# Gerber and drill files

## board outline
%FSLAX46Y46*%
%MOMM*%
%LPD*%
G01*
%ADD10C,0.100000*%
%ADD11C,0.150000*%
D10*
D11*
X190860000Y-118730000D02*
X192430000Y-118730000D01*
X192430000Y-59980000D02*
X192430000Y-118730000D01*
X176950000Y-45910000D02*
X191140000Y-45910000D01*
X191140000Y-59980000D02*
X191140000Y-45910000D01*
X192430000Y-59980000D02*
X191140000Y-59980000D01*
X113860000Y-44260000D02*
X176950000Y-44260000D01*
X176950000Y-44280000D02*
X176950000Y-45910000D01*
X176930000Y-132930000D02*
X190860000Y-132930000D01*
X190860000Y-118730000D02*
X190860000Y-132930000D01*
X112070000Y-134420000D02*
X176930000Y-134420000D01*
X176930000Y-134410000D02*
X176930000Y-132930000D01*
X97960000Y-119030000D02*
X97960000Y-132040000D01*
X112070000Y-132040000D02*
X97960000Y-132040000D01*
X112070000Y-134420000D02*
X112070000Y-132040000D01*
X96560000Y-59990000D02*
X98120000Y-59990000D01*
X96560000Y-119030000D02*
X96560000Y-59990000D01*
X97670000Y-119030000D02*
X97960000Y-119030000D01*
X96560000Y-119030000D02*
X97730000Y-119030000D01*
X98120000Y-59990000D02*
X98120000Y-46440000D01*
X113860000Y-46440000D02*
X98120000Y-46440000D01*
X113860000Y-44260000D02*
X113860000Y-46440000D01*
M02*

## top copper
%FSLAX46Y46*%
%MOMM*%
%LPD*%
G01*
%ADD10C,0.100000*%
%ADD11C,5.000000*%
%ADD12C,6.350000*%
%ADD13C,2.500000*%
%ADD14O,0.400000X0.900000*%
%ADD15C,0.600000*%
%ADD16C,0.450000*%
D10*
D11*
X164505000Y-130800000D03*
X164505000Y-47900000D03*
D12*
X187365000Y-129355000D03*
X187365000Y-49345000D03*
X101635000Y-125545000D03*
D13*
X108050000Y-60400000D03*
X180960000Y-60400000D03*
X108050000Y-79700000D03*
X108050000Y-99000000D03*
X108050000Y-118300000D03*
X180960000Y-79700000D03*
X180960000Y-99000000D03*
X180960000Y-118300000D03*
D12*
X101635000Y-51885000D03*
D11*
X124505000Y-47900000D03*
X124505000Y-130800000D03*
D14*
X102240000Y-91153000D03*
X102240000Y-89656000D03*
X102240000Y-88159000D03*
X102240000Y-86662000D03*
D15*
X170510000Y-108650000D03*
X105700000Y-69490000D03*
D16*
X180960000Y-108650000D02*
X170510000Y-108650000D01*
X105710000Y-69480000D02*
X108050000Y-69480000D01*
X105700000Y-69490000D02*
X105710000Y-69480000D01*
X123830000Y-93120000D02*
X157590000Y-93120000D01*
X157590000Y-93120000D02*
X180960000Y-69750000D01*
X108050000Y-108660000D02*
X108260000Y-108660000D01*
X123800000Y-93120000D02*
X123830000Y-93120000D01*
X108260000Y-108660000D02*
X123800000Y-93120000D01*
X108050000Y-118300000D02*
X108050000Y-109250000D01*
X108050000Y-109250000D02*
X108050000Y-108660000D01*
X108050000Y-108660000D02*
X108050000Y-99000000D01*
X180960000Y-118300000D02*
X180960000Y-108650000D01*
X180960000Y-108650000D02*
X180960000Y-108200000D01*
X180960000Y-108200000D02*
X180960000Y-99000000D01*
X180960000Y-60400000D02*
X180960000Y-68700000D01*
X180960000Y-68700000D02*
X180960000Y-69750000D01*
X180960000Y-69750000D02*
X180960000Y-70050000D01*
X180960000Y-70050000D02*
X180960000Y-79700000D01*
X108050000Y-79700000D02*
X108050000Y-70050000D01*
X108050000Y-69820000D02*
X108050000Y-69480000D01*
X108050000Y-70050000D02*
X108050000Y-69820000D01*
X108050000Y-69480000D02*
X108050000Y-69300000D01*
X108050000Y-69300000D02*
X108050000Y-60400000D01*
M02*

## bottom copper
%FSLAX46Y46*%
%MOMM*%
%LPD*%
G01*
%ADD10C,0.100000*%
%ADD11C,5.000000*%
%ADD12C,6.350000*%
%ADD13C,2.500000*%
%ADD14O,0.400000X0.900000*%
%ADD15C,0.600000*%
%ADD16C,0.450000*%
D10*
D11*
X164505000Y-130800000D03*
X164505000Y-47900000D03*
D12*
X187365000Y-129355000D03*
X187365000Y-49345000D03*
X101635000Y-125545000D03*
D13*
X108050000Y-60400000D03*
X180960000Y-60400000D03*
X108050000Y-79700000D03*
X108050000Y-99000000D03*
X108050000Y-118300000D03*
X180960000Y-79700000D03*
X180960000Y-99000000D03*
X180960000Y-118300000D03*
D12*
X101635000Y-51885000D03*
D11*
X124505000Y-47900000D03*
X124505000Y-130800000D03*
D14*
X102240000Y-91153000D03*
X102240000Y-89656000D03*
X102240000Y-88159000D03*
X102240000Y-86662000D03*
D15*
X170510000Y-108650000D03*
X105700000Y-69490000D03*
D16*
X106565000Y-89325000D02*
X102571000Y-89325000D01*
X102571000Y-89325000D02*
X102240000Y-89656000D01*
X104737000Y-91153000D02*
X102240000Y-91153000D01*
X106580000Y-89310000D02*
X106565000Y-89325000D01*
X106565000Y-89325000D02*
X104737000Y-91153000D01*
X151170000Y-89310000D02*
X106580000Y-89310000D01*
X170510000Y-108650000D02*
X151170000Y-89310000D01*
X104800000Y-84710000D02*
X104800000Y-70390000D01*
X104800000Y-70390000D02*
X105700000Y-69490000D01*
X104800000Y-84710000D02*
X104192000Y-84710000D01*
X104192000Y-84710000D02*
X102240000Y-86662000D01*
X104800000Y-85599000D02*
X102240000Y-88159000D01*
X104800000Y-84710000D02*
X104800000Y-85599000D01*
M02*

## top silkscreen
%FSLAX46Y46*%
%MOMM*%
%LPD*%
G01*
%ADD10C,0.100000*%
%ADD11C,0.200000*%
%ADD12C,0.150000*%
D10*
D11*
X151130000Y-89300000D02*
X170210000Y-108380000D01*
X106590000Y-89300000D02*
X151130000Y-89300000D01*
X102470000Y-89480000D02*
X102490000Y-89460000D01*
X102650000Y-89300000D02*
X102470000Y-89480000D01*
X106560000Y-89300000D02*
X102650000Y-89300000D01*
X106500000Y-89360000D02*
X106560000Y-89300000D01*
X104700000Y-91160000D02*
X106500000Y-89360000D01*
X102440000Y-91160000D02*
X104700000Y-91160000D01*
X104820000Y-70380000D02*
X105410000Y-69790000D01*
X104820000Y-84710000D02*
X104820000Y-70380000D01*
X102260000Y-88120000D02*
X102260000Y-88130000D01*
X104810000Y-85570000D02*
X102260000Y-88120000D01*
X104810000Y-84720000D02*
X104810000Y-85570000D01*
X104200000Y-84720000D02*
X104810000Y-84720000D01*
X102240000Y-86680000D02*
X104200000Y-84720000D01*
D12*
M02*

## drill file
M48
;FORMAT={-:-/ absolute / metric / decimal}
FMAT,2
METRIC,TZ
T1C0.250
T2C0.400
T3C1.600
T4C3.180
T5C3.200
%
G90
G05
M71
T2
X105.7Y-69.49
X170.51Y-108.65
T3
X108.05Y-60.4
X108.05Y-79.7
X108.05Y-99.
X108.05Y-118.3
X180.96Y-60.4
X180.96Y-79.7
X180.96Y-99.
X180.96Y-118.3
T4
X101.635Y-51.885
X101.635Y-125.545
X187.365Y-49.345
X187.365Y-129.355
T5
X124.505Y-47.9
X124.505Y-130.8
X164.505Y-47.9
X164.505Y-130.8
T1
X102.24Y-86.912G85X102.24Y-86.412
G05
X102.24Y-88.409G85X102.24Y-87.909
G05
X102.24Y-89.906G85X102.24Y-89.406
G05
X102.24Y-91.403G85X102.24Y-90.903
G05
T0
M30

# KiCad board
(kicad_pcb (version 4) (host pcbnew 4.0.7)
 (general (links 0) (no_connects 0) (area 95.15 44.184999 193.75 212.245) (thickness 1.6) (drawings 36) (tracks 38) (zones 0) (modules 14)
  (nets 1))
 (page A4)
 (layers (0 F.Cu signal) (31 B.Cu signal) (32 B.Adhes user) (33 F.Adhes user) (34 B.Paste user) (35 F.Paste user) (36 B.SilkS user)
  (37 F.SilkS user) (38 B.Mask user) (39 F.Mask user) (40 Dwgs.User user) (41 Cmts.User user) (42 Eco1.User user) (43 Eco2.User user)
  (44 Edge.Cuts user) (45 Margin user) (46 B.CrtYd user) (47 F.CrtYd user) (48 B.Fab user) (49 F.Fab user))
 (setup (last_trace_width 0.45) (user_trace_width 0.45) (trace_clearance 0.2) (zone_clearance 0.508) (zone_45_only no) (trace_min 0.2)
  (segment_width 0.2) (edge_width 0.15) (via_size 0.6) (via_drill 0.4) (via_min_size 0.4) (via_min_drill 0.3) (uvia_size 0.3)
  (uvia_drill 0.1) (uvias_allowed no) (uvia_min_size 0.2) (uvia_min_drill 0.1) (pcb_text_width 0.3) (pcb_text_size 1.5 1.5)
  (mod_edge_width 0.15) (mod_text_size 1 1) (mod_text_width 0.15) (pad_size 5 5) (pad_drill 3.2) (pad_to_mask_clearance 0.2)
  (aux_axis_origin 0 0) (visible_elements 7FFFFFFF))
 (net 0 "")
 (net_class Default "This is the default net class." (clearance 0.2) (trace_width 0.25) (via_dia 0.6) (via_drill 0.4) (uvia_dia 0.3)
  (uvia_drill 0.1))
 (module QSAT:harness (layer F.Cu) (at 163.19 210.67)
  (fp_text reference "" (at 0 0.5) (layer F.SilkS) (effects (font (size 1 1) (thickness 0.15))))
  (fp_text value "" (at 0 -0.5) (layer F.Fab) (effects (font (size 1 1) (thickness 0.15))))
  (pad 1 thru_hole circle (at 1.315 -79.87) (size 5 5) (drill 3.2) (layers *.Cu *.Mask)))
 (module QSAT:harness (layer F.Cu) (at 164.505 48.28)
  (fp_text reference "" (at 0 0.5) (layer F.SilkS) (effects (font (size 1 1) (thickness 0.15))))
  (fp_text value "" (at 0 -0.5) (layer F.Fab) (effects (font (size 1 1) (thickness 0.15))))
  (pad 1 thru_hole circle (at 0 -0.38) (size 5 5) (drill 3.2) (layers *.Cu *.Mask)))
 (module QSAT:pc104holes (layer F.Cu) (at 187.555 129.705)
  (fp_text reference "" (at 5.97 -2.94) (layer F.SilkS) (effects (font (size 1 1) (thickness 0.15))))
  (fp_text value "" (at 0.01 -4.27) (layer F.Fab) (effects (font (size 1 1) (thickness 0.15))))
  (pad 1 thru_hole circle (at -0.19 -0.35) (size 6.35 6.35) (drill 3.18) (layers *.Cu *.Mask)))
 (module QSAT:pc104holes (layer F.Cu) (at 187.565 49.585)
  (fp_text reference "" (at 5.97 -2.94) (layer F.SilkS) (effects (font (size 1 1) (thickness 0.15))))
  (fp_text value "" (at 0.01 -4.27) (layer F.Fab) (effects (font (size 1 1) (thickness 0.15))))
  (pad 1 thru_hole circle (at -0.2 -0.24) (size 6.35 6.35) (drill 3.18) (layers *.Cu *.Mask)))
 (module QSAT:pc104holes (layer F.Cu) (at 101.975 129.815)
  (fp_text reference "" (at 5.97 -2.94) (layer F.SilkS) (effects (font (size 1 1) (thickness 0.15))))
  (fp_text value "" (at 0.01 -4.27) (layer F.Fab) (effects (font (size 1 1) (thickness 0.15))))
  (pad 1 thru_hole circle (at -0.34 -4.27) (size 6.35 6.35) (drill 3.18) (layers *.Cu *.Mask)))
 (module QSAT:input (layer F.Cu) (at 193.3 99.4)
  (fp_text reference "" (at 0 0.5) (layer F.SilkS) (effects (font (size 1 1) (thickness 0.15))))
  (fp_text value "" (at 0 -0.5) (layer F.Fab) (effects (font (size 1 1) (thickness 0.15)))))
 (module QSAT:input (layer F.Cu) (at 193.2 113.7)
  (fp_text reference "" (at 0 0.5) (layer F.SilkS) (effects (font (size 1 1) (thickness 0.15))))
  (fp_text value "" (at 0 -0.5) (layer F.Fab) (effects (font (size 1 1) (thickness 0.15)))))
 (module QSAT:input (layer F.Cu) (at 95.6 75.3)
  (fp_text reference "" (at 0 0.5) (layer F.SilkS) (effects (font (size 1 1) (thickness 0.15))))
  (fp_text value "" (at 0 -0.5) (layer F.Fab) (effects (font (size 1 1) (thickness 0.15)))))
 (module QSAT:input (layer F.Cu) (at 95.7 60.9)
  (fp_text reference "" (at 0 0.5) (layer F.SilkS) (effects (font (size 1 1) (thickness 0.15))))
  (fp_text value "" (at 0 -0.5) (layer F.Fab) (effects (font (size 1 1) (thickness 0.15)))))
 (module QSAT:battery (layer F.Cu) (at 116.7 60.4)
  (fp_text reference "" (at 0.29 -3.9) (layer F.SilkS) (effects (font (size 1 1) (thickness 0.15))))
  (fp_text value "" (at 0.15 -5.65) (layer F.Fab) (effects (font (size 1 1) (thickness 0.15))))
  (pad 2 thru_hole circle (at -8.65 0) (size 2.5 2.5) (drill 1.6) (layers *.Cu *.Mask))
  (pad 4 thru_hole circle (at 64.26 0) (size 2.5 2.5) (drill 1.6) (layers *.Cu *.Mask))
  (pad 10 thru_hole circle (at -8.65 19.3) (size 2.5 2.5) (drill 1.6) (layers *.Cu *.Mask))
  (pad 11 thru_hole circle (at -8.65 38.6) (size 2.5 2.5) (drill 1.6) (layers *.Cu *.Mask))
  (pad 12 thru_hole circle (at -8.65 57.9) (size 2.5 2.5) (drill 1.6) (layers *.Cu *.Mask))
  (pad 13 thru_hole circle (at 64.26 19.3) (size 2.5 2.5) (drill 1.6) (layers *.Cu *.Mask))
  (pad 14 thru_hole circle (at 64.26 38.6) (size 2.5 2.5) (drill 1.6) (layers *.Cu *.Mask))
  (pad 15 thru_hole circle (at 64.26 57.9) (size 2.5 2.5) (drill 1.6) (layers *.Cu *.Mask)))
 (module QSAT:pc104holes (layer F.Cu) (at 101.635 51.885)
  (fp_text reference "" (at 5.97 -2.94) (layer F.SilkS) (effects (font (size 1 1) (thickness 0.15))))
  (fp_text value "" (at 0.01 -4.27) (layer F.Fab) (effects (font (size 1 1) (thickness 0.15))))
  (pad 1 thru_hole circle (at 0 0) (size 6.35 6.35) (drill 3.18) (layers *.Cu *.Mask)))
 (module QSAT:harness (layer F.Cu) (at 124.505 47.9)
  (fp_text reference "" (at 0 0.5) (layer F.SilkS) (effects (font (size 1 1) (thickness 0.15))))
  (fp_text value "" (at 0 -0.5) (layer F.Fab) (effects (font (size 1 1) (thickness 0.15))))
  (pad 1 thru_hole circle (at 0 0) (size 5 5) (drill 3.2) (layers *.Cu *.Mask)))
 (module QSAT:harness (layer F.Cu) (at 124.505 130.8)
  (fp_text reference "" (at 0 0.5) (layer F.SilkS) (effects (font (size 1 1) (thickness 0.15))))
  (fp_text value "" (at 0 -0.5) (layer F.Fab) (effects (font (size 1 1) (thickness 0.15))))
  (pad 1 thru_hole circle (at 0 0) (size 5 5) (drill 3.2) (layers *.Cu *.Mask)))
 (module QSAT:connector (layer F.Cu) (at 102.24 88.9 90)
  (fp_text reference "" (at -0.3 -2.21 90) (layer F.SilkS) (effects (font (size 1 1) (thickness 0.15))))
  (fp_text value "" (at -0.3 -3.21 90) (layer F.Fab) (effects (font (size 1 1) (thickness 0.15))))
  (pad 21 thru_hole oval (at -2.253 0 90) (size 0.9 0.4) (drill oval 0.75 0.25) (layers *.Cu *.Mask))
  (pad 31 thru_hole oval (at -0.756 0 90) (size 0.9 0.4) (drill oval 0.75 0.25) (layers *.Cu *.Mask))
  (pad 41 thru_hole oval (at 0.741 0 90) (size 0.9 0.4) (drill oval 0.75 0.25) (layers *.Cu *.Mask))
  (pad 51 thru_hole oval (at 2.238 0 90) (size 0.9 0.4) (drill oval 0.75 0.25) (layers *.Cu *.Mask)))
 (gr_line (start 151.13 89.3) (end 170.21 108.38) (angle 90) (layer F.SilkS) (width 0.2))
 (gr_line (start 106.59 89.3) (end 151.13 89.3) (angle 90) (layer F.SilkS) (width 0.2))
 (gr_line (start 102.47 89.48) (end 102.49 89.46) (angle 90) (layer F.SilkS) (width 0.2))
 (gr_line (start 102.65 89.3) (end 102.47 89.48) (angle 90) (layer F.SilkS) (width 0.2))
 (gr_line (start 106.56 89.3) (end 102.65 89.3) (angle 90) (layer F.SilkS) (width 0.2))
 (gr_line (start 106.5 89.36) (end 106.56 89.3) (angle 90) (layer F.SilkS) (width 0.2))
 (gr_line (start 104.7 91.16) (end 106.5 89.36) (angle 90) (layer F.SilkS) (width 0.2))
 (gr_line (start 102.44 91.16) (end 104.7 91.16) (angle 90) (layer F.SilkS) (width 0.2))
 (gr_line (start 104.82 70.38) (end 105.41 69.79) (angle 90) (layer F.SilkS) (width 0.2))
 (gr_line (start 104.82 84.71) (end 104.82 70.38) (angle 90) (layer F.SilkS) (width 0.2))
 (gr_line (start 102.26 88.12) (end 102.26 88.13) (angle 90) (layer F.SilkS) (width 0.2))
 (gr_line (start 104.81 85.57) (end 102.26 88.12) (angle 90) (layer F.SilkS) (width 0.2))
 (gr_line (start 104.81 84.72) (end 104.81 85.57) (angle 90) (layer F.SilkS) (width 0.2))
 (gr_line (start 104.2 84.72) (end 104.81 84.72) (angle 90) (layer F.SilkS) (width 0.2))
 (gr_line (start 102.24 86.68) (end 104.2 84.72) (angle 90) (layer F.SilkS) (width 0.2))
 (gr_line (start 190.86 118.73) (end 192.43 118.73) (angle 90) (layer Edge.Cuts) (width 0.15))
 (gr_line (start 192.43 59.98) (end 192.43 118.73) (angle 90) (layer Edge.Cuts) (width 0.15))
 (gr_line (start 176.95 45.91) (end 191.14 45.91) (angle 90) (layer Edge.Cuts) (width 0.15))
 (gr_line (start 191.14 59.98) (end 191.14 45.91) (angle 90) (layer Edge.Cuts) (width 0.15))
 (gr_line (start 192.43 59.98) (end 191.14 59.98) (angle 90) (layer Edge.Cuts) (width 0.15))
 (gr_line (start 113.86 44.26) (end 176.95 44.26) (angle 90) (layer Edge.Cuts) (width 0.15))
 (gr_line (start 176.95 44.28) (end 176.95 45.91) (angle 90) (layer Edge.Cuts) (width 0.15))
 (gr_line (start 176.93 132.93) (end 190.86 132.93) (angle 90) (layer Edge.Cuts) (width 0.15))
 (gr_line (start 190.86 118.73) (end 190.86 132.93) (angle 90) (layer Edge.Cuts) (width 0.15))
 (gr_line (start 112.07 134.42) (end 176.93 134.42) (angle 90) (layer Edge.Cuts) (width 0.15))
 (gr_line (start 176.93 134.41) (end 176.93 132.93) (angle 90) (layer Edge.Cuts) (width 0.15))
 (gr_line (start 97.96 119.03) (end 97.96 132.04) (angle 90) (layer Edge.Cuts) (width 0.15))
 (gr_line (start 112.07 132.04) (end 97.96 132.04) (angle 90) (layer Edge.Cuts) (width 0.15))
 (gr_line (start 112.07 134.42) (end 112.07 132.04) (angle 90) (layer Edge.Cuts) (width 0.15))
 (gr_line (start 96.56 59.99) (end 98.12 59.99) (angle 90) (layer Edge.Cuts) (width 0.15))
 (gr_line (start 96.56 119.03) (end 96.56 59.99) (angle 90) (layer Edge.Cuts) (width 0.15))
 (gr_line (start 97.67 119.03) (end 97.96 119.03) (angle 90) (layer Edge.Cuts) (width 0.15))
 (gr_line (start 96.56 119.03) (end 97.73 119.03) (angle 90) (layer Edge.Cuts) (width 0.15))
 (gr_line (start 98.12 59.99) (end 98.12 46.44) (angle 90) (layer Edge.Cuts) (width 0.15))
 (gr_line (start 113.86 46.44) (end 98.12 46.44) (angle 90) (layer Edge.Cuts) (width 0.15))
 (gr_line (start 113.86 44.26) (end 113.86 46.44) (angle 90) (layer Edge.Cuts) (width 0.15))
 (segment (start 106.565 89.325) (end 102.571 89.325) (width 0.45) (layer B.Cu) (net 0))
 (segment (start 102.571 89.325) (end 102.24 89.656) (width 0.45) (layer B.Cu) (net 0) (status 800000))
 (segment (start 180.96 108.65) (end 170.51 108.65) (width 0.45) (layer F.Cu) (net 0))
 (segment (start 104.737 91.153) (end 102.24 91.153) (width 0.45) (layer B.Cu) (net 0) (status 800000))
 (segment (start 106.58 89.31) (end 106.565 89.325) (width 0.45) (layer B.Cu) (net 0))
 (segment (start 106.565 89.325) (end 104.737 91.153) (width 0.45) (layer B.Cu) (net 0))
 (segment (start 151.17 89.31) (end 106.58 89.31) (width 0.45) (layer B.Cu) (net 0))
 (segment (start 170.51 108.65) (end 151.17 89.31) (width 0.45) (layer B.Cu) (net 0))
 (via (at 170.51 108.65) (size 0.6) (drill 0.4) (layers F.Cu B.Cu) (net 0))
 (segment (start 104.8 84.71) (end 104.8 70.39) (width 0.45) (layer B.Cu) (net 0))
 (segment (start 105.71 69.48) (end 108.05 69.48) (width 0.45) (layer F.Cu) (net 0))
 (segment (start 105.7 69.49) (end 105.71 69.48) (width 0.45) (layer F.Cu) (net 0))
 (via (at 105.7 69.49) (size 0.6) (drill 0.4) (layers F.Cu B.Cu) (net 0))
 (segment (start 104.8 70.39) (end 105.7 69.49) (width 0.45) (layer B.Cu) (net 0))
 (segment (start 104.8 84.71) (end 104.192 84.71) (width 0.45) (layer B.Cu) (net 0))
 (segment (start 104.192 84.71) (end 102.24 86.662) (width 0.45) (layer B.Cu) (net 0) (status 800000))
 (segment (start 104.8 85.599) (end 102.24 88.159) (width 0.45) (layer B.Cu) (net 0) (status 800000))
 (segment (start 104.8 84.71) (end 104.8 85.599) (width 0.45) (layer B.Cu) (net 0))
 (segment (start 123.83 93.12) (end 157.59 93.12) (width 0.45) (layer F.Cu) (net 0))
 (segment (start 157.59 93.12) (end 180.96 69.75) (width 0.45) (layer F.Cu) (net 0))
 (segment (start 108.05 108.66) (end 108.26 108.66) (width 0.45) (layer F.Cu) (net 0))
 (segment (start 123.8 93.12) (end 123.83 93.12) (width 0.45) (layer F.Cu) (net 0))
 (segment (start 108.26 108.66) (end 123.8 93.12) (width 0.45) (layer F.Cu) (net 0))
 (segment (start 108.05 118.3) (end 108.05 109.25) (width 0.45) (layer F.Cu) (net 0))
 (segment (start 108.05 109.25) (end 108.05 108.66) (width 0.45) (layer F.Cu) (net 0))
 (segment (start 108.05 108.66) (end 108.05 99) (width 0.45) (layer F.Cu) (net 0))
 (segment (start 180.96 118.3) (end 180.96 108.65) (width 0.45) (layer F.Cu) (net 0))
 (segment (start 180.96 108.65) (end 180.96 108.2) (width 0.45) (layer F.Cu) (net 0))
 (segment (start 180.96 108.2) (end 180.96 99) (width 0.45) (layer F.Cu) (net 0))
 (segment (start 180.96 60.4) (end 180.96 68.7) (width 0.45) (layer F.Cu) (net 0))
 (segment (start 180.96 68.7) (end 180.96 69.75) (width 0.45) (layer F.Cu) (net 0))
 (segment (start 180.96 69.75) (end 180.96 70.05) (width 0.45) (layer F.Cu) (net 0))
 (segment (start 180.96 70.05) (end 180.96 79.7) (width 0.45) (layer F.Cu) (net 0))
 (segment (start 108.05 79.7) (end 108.05 70.05) (width 0.45) (layer F.Cu) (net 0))
 (segment (start 108.05 69.82) (end 108.05 69.48) (width 0.45) (layer F.Cu) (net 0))
 (segment (start 108.05 70.05) (end 108.05 69.82) (width 0.45) (layer F.Cu) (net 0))
 (segment (start 108.05 69.48) (end 108.05 69.3) (width 0.45) (layer F.Cu) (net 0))
 (segment (start 108.05 69.3) (end 108.05 60.4) (width 0.45) (layer F.Cu) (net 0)))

